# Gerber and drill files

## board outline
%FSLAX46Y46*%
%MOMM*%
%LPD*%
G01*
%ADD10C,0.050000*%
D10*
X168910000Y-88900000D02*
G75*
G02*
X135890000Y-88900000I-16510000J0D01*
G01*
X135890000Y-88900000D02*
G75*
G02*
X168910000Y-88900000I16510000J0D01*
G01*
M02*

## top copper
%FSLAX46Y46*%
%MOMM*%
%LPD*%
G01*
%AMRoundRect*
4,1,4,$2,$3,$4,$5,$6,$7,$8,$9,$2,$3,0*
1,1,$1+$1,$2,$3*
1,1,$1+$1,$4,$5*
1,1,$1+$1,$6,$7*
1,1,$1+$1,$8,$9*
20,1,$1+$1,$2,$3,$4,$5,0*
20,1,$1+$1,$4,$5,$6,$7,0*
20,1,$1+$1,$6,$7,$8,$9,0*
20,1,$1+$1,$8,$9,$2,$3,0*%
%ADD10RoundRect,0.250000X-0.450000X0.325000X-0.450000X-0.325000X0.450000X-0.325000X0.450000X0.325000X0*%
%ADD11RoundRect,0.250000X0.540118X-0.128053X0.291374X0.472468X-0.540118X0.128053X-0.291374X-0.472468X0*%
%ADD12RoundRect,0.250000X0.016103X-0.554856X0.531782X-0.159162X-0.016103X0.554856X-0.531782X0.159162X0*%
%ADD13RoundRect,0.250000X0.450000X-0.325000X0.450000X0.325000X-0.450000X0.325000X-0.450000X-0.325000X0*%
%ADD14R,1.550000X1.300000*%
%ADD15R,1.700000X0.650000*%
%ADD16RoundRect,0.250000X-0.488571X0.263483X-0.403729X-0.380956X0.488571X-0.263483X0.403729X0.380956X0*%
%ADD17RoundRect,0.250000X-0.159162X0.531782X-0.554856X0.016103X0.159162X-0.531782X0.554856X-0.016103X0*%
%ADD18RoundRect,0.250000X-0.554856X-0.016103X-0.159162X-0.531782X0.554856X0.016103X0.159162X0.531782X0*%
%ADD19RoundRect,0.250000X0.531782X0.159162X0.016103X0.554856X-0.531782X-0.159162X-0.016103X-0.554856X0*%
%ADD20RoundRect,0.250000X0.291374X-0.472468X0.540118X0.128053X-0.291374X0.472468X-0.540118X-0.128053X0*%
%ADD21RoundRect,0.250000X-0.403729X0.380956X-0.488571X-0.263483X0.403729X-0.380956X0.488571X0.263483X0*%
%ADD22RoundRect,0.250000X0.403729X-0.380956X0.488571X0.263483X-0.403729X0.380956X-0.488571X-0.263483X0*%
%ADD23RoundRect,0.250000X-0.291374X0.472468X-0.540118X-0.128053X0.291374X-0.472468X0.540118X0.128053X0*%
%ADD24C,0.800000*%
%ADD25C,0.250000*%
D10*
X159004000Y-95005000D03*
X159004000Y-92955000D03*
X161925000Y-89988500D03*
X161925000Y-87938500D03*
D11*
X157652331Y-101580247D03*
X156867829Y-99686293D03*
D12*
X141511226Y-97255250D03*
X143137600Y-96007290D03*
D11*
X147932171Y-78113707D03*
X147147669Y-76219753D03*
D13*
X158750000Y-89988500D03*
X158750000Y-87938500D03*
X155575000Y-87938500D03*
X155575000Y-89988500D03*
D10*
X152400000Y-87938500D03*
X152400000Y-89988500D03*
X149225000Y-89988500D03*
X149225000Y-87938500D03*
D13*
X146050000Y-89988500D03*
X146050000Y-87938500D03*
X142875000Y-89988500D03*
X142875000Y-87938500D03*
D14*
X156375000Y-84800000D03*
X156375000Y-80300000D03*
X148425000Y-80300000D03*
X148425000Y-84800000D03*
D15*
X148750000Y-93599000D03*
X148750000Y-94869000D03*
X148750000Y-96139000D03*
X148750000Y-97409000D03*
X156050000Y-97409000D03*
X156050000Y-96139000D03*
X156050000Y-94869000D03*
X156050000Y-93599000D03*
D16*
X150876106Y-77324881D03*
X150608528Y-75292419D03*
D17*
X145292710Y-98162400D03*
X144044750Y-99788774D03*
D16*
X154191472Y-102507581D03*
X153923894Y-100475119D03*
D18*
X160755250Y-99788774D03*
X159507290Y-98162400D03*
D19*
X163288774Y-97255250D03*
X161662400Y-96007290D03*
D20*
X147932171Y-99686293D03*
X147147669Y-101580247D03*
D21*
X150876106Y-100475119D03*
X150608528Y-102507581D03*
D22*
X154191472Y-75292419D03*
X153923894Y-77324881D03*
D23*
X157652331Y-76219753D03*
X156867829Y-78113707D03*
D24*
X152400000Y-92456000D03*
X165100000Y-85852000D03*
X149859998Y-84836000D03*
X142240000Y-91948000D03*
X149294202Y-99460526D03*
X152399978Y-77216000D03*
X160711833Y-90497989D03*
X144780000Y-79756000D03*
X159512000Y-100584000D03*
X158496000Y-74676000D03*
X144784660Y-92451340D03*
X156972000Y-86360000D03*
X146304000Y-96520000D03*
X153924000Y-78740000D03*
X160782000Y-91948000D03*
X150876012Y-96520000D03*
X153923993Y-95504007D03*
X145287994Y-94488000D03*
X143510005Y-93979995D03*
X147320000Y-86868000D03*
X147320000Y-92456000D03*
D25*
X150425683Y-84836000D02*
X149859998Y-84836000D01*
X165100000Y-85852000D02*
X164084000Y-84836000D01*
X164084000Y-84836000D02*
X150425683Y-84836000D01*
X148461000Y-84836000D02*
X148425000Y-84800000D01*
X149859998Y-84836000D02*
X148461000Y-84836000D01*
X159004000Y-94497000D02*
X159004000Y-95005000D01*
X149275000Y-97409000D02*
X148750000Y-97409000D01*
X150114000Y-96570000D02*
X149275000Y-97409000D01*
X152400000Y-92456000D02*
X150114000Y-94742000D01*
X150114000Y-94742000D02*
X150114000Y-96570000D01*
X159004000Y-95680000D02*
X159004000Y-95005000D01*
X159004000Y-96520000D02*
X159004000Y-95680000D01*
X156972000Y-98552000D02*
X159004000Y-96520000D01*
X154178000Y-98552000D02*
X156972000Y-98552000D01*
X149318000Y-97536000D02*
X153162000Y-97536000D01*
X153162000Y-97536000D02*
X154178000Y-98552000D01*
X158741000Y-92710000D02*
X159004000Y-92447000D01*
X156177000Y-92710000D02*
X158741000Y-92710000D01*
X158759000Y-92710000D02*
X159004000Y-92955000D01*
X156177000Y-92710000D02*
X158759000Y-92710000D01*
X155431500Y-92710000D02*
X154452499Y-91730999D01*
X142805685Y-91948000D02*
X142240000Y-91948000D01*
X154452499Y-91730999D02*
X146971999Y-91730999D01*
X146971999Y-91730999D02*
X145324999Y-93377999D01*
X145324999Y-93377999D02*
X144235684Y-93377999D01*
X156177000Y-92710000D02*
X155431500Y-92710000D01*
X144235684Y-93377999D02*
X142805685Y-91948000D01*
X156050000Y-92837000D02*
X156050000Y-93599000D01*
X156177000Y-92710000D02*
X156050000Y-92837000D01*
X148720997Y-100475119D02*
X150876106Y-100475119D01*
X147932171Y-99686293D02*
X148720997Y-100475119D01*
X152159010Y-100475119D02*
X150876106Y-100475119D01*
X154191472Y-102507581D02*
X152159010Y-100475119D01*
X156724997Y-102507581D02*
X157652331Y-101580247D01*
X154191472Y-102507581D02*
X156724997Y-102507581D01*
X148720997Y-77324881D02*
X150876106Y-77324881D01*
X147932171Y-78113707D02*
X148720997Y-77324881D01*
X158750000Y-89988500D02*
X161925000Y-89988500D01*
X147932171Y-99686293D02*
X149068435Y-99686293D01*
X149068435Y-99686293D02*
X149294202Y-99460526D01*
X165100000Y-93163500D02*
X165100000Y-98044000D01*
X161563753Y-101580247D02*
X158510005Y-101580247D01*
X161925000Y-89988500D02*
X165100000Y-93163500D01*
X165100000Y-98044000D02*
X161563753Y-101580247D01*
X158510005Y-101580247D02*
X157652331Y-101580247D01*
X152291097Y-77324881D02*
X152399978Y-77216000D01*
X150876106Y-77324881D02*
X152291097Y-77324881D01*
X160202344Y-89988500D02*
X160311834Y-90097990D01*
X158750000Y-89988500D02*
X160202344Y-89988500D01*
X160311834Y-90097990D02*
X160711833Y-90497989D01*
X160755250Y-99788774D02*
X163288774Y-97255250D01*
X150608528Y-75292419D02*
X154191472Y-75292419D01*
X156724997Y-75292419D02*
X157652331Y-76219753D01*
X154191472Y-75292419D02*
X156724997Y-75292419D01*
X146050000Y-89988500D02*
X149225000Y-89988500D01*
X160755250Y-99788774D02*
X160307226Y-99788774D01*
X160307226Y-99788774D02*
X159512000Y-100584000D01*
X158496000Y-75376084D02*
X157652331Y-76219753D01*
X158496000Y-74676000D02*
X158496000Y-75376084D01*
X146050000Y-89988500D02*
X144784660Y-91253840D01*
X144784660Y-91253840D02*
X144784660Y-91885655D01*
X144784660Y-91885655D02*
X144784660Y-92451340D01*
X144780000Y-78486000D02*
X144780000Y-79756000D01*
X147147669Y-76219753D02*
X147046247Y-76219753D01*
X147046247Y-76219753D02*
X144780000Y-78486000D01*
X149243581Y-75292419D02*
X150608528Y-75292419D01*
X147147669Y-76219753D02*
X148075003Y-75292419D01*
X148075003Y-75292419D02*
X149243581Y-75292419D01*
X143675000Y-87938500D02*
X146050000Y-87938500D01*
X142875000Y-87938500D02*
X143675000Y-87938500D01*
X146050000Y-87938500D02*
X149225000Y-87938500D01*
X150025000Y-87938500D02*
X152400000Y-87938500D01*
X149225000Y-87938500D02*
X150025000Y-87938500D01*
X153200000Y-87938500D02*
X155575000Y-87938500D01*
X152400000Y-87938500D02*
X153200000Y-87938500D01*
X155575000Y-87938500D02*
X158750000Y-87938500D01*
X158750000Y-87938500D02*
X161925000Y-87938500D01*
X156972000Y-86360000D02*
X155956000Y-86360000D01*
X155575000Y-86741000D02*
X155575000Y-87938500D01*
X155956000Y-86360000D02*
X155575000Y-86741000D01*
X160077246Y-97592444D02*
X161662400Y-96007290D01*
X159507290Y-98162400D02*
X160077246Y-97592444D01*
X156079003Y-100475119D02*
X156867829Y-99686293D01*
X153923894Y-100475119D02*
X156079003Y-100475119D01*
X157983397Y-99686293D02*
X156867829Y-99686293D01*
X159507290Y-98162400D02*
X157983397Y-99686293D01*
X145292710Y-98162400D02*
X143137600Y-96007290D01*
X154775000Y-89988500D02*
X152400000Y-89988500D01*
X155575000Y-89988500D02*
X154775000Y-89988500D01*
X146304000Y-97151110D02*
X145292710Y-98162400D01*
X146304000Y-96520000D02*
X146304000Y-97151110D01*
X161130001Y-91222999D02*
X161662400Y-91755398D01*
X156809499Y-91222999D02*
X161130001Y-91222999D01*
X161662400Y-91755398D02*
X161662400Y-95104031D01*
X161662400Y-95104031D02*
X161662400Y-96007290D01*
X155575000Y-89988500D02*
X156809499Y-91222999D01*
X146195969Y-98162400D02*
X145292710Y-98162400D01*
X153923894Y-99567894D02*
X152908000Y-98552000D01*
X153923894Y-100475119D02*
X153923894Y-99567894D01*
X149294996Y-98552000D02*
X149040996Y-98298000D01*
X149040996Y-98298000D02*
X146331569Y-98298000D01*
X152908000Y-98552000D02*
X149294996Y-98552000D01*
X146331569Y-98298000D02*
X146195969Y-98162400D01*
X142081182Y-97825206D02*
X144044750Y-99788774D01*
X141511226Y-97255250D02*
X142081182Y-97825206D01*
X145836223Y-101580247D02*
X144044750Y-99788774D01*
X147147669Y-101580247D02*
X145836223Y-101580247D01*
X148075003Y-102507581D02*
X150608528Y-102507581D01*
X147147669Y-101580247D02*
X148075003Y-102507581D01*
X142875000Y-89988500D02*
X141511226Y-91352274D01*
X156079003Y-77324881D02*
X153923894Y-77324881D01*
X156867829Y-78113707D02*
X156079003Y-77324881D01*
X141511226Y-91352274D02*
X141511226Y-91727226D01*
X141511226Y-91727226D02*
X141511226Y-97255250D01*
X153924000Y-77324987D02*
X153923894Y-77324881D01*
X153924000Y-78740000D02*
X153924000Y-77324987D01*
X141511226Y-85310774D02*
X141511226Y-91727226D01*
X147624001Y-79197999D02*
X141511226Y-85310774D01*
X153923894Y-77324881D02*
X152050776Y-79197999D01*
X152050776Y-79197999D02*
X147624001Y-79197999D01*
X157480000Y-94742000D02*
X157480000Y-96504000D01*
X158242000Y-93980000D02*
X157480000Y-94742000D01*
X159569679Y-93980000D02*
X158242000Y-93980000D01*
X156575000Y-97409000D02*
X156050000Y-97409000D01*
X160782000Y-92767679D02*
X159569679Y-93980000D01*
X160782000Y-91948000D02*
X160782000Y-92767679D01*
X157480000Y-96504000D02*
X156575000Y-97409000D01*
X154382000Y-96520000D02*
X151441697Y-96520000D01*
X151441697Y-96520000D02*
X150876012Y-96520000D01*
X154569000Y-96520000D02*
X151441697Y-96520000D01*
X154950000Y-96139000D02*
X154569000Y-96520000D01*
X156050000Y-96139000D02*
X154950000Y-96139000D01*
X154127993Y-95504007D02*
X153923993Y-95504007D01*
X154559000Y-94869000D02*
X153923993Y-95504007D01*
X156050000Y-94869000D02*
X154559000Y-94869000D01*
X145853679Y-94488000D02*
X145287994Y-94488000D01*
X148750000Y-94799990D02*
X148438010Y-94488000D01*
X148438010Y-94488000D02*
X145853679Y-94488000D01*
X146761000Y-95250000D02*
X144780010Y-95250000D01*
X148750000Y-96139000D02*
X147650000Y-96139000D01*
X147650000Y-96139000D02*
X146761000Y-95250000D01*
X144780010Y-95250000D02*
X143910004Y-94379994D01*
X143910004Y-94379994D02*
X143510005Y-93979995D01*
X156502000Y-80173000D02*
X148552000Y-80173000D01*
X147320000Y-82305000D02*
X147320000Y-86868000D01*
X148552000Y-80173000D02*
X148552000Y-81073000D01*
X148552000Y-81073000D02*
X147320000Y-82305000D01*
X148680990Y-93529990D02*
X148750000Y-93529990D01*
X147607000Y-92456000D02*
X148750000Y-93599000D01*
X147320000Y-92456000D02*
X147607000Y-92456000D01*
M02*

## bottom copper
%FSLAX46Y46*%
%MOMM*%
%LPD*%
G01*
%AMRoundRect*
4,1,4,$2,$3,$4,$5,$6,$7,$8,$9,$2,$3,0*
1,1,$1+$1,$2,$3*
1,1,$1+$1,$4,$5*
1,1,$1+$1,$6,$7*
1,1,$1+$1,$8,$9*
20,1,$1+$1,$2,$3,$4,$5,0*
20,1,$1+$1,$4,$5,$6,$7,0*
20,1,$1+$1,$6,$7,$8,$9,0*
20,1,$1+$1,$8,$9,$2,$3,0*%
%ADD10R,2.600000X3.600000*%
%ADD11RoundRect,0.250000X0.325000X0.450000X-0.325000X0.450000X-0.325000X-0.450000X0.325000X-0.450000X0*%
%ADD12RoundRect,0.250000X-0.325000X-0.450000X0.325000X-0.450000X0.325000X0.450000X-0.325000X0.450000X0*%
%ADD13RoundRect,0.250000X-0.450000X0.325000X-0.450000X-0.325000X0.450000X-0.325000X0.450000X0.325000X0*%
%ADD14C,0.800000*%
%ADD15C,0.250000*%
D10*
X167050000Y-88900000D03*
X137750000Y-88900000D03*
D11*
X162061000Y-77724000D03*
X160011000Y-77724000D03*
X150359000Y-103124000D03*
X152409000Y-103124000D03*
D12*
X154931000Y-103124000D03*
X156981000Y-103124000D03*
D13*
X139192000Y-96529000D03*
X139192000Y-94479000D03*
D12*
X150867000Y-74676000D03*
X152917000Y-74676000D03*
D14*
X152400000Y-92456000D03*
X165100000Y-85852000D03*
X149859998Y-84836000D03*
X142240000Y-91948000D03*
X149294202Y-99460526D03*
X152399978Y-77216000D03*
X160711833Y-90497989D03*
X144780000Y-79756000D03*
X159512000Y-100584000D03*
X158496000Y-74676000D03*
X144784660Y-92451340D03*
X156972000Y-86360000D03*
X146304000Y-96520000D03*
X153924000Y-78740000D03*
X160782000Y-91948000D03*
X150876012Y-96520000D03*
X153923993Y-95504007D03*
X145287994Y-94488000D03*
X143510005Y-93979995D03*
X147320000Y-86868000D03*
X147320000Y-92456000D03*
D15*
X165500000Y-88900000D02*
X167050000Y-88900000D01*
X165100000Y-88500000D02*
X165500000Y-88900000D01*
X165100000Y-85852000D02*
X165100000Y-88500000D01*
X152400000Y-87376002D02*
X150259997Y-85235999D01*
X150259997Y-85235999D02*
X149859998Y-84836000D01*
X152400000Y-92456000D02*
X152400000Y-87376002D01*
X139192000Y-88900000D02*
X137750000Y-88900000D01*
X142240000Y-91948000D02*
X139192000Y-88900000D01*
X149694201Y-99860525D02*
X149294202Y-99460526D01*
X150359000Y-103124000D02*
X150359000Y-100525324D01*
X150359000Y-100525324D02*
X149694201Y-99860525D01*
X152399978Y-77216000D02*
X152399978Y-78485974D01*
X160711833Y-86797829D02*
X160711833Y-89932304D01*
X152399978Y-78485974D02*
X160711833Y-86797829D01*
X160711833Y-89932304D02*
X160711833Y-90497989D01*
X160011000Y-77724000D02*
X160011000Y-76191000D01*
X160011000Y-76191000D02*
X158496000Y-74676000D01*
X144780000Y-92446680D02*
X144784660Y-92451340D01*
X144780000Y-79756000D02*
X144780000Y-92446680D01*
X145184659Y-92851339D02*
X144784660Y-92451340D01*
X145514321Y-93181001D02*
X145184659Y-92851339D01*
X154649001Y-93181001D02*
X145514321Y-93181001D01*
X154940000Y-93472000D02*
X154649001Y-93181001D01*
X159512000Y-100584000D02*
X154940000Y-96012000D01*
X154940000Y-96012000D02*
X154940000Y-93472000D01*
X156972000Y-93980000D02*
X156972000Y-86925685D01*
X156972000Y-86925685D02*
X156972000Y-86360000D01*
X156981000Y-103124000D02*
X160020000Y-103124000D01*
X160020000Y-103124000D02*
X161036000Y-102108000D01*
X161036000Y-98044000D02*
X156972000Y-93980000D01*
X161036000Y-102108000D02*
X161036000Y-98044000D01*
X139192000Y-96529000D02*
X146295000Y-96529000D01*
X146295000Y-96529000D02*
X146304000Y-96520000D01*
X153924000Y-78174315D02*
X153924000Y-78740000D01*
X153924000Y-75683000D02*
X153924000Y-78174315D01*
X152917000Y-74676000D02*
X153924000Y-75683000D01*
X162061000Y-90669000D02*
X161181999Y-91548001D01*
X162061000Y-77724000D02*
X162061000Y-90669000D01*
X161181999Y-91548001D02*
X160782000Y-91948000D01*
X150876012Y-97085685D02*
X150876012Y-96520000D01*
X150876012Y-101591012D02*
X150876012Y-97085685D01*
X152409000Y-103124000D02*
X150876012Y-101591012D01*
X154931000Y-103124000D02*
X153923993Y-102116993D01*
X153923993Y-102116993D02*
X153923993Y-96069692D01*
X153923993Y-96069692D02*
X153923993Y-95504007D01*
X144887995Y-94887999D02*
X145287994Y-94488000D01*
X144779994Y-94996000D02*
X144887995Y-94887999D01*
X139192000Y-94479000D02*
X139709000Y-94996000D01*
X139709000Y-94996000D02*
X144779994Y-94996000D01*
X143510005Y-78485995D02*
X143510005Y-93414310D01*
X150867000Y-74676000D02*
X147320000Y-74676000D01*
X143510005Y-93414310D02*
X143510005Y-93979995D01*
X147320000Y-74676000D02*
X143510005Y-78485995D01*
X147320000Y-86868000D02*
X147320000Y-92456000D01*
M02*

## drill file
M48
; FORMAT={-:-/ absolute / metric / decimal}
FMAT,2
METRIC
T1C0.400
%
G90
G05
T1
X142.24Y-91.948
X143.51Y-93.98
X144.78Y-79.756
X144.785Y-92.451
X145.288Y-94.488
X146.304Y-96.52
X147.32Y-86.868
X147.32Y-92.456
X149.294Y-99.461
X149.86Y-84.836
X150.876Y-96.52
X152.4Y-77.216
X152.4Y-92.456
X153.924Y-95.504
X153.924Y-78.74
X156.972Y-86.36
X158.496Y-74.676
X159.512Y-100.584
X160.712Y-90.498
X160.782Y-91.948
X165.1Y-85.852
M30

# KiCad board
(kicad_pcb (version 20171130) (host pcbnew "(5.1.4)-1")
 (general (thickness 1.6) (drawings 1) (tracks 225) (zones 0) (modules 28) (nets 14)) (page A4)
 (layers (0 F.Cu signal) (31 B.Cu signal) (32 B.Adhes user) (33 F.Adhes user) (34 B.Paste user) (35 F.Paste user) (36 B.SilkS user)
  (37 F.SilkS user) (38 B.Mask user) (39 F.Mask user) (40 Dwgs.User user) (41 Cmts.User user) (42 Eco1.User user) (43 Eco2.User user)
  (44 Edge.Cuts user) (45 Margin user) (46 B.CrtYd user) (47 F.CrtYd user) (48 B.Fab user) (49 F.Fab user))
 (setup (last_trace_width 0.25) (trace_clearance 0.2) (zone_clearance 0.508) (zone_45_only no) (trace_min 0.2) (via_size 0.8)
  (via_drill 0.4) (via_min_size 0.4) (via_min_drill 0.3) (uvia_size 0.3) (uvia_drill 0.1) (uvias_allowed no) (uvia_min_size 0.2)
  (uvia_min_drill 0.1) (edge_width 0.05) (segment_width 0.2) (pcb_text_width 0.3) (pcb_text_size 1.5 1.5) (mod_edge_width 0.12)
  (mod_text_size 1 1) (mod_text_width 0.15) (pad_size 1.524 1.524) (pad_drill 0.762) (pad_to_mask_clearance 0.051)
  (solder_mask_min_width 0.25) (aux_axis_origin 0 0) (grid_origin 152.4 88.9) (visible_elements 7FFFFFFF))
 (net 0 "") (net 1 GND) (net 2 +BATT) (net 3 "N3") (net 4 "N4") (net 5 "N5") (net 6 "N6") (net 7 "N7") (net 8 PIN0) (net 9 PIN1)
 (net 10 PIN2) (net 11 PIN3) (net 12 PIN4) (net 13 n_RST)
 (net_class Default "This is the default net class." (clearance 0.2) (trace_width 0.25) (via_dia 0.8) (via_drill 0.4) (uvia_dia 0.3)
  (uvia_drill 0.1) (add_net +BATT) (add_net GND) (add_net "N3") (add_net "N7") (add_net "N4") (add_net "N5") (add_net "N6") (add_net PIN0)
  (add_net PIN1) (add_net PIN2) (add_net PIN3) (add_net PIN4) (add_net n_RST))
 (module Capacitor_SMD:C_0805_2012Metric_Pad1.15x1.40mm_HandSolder (layer F.Cu) (at 159.004 93.98 270)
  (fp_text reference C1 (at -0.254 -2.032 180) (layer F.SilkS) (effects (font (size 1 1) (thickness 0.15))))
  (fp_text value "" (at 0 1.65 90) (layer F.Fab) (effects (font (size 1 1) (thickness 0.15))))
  (pad 2 smd roundrect (at 1.025 0 270) (size 1.15 1.4) (layers F.Cu F.Paste F.Mask) (roundrect_rratio 0.217391) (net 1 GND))
  (pad 1 smd roundrect (at -1.025 0 270) (size 1.15 1.4) (layers F.Cu F.Paste F.Mask) (roundrect_rratio 0.217391) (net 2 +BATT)))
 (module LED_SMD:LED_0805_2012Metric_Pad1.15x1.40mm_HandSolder (layer F.Cu) (at 161.925 88.9635 270)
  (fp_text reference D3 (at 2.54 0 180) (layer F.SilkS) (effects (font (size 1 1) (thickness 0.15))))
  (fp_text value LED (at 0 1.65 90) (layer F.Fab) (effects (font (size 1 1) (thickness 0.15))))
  (pad 2 smd roundrect (at 1.025 0 270) (size 1.15 1.4) (layers F.Cu F.Paste F.Mask) (roundrect_rratio 0.217391) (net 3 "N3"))
  (pad 1 smd roundrect (at -1.025 0 270) (size 1.15 1.4) (layers F.Cu F.Paste F.Mask) (roundrect_rratio 0.217391) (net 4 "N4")))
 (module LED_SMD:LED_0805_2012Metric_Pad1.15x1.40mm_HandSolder (layer F.Cu) (at 157.26008 100.63327 112.5)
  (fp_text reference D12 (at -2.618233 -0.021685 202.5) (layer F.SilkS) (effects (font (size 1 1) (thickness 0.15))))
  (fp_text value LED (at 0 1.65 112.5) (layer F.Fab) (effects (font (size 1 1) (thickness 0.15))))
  (pad 1 smd roundrect (at -1.025 0 112.5) (size 1.15 1.4) (layers F.Cu F.Paste F.Mask) (roundrect_rratio 0.217391) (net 3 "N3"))
  (pad 2 smd roundrect (at 1.025 0 112.5) (size 1.15 1.4) (layers F.Cu F.Paste F.Mask) (roundrect_rratio 0.217391) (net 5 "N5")))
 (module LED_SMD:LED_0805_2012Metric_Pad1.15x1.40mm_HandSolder (layer F.Cu) (at 142.324413 96.63127 37.5)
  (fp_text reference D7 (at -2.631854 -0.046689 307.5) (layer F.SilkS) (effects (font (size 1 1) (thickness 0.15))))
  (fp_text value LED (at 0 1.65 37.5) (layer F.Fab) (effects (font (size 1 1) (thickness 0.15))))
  (pad 1 smd roundrect (at -1.025 0 37.5) (size 1.15 1.4) (layers F.Cu F.Paste F.Mask) (roundrect_rratio 0.217391) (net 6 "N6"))
  (pad 2 smd roundrect (at 1.025 0 37.5) (size 1.15 1.4) (layers F.Cu F.Paste F.Mask) (roundrect_rratio 0.217391) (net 5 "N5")))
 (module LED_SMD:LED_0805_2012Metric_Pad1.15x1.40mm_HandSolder (layer F.Cu) (at 147.53992 77.16673 112.5)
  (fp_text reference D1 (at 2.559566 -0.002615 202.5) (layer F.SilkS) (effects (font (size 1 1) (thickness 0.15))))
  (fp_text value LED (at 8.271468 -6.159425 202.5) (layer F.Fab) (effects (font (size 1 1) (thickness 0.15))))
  (pad 1 smd roundrect (at -1.025 0 112.5) (size 1.15 1.4) (layers F.Cu F.Paste F.Mask) (roundrect_rratio 0.217391) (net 3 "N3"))
  (pad 2 smd roundrect (at 1.025 0 112.5) (size 1.15 1.4) (layers F.Cu F.Paste F.Mask) (roundrect_rratio 0.217391) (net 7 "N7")))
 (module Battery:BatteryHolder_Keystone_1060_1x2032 (layer B.Cu) (at 152.4 88.9)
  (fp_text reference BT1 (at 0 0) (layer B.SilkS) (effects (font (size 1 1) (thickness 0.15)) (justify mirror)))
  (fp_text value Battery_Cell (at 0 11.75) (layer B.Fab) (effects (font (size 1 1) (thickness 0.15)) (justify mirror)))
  (pad 2 smd rect (at 14.65 0 180) (size 2.6 3.6) (layers B.Cu B.Paste B.Mask) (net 1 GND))
  (pad 1 smd rect (at -14.65 0 180) (size 2.6 3.6) (layers B.Cu B.Paste B.Mask) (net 2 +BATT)))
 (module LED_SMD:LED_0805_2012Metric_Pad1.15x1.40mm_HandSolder (layer F.Cu) (at 158.75 88.9635 90)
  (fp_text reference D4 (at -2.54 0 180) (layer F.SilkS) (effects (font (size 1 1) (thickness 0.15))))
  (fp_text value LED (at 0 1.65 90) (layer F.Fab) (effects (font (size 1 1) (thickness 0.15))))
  (pad 1 smd roundrect (at -1.025 0 90) (size 1.15 1.4) (layers F.Cu F.Paste F.Mask) (roundrect_rratio 0.217391) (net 3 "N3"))
  (pad 2 smd roundrect (at 1.025 0 90) (size 1.15 1.4) (layers F.Cu F.Paste F.Mask) (roundrect_rratio 0.217391) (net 4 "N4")))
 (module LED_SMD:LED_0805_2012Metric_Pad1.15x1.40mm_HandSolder (layer F.Cu) (at 155.575 88.9635 90)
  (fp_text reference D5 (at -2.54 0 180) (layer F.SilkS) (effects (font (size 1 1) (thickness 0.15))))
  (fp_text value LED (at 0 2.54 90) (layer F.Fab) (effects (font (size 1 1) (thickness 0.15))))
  (pad 2 smd roundrect (at 1.025 0 90) (size 1.15 1.4) (layers F.Cu F.Paste F.Mask) (roundrect_rratio 0.217391) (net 4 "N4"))
  (pad 1 smd roundrect (at -1.025 0 90) (size 1.15 1.4) (layers F.Cu F.Paste F.Mask) (roundrect_rratio 0.217391) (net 5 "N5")))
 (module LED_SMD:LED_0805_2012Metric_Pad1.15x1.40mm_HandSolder (layer F.Cu) (at 152.4 88.9635 270)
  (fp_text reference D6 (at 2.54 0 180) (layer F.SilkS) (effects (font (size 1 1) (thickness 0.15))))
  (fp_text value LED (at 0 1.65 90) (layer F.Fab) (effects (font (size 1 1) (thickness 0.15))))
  (pad 1 smd roundrect (at -1.025 0 270) (size 1.15 1.4) (layers F.Cu F.Paste F.Mask) (roundrect_rratio 0.217391) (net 4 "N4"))
  (pad 2 smd roundrect (at 1.025 0 270) (size 1.15 1.4) (layers F.Cu F.Paste F.Mask) (roundrect_rratio 0.217391) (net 5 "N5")))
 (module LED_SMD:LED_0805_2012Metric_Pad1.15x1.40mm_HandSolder (layer F.Cu) (at 149.225 88.9635 270)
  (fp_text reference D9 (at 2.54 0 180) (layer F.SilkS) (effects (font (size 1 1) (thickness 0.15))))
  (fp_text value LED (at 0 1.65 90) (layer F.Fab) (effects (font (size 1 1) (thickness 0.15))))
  (pad 2 smd roundrect (at 1.025 0 270) (size 1.15 1.4) (layers F.Cu F.Paste F.Mask) (roundrect_rratio 0.217391) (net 7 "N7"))
  (pad 1 smd roundrect (at -1.025 0 270) (size 1.15 1.4) (layers F.Cu F.Paste F.Mask) (roundrect_rratio 0.217391) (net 4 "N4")))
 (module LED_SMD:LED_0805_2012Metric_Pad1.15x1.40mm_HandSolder (layer F.Cu) (at 146.05 88.9635 90)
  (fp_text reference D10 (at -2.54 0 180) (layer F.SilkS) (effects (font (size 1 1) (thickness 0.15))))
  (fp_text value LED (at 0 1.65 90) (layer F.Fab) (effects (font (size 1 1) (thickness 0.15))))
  (pad 1 smd roundrect (at -1.025 0 90) (size 1.15 1.4) (layers F.Cu F.Paste F.Mask) (roundrect_rratio 0.217391) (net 7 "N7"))
  (pad 2 smd roundrect (at 1.025 0 90) (size 1.15 1.4) (layers F.Cu F.Paste F.Mask) (roundrect_rratio 0.217391) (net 4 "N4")))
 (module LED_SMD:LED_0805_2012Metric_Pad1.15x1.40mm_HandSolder (layer F.Cu) (at 142.875 88.9635 90)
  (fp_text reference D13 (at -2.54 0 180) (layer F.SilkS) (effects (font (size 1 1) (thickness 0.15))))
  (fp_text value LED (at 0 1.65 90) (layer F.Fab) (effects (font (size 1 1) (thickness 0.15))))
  (pad 1 smd roundrect (at -1.025 0 90) (size 1.15 1.4) (layers F.Cu F.Paste F.Mask) (roundrect_rratio 0.217391) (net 6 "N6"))
  (pad 2 smd roundrect (at 1.025 0 90) (size 1.15 1.4) (layers F.Cu F.Paste F.Mask) (roundrect_rratio 0.217391) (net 4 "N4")))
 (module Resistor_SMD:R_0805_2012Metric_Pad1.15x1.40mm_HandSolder (layer B.Cu) (at 161.036 77.724 180)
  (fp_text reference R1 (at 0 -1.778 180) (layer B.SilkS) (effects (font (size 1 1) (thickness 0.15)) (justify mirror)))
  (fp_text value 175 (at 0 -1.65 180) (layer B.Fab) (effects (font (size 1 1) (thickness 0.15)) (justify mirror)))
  (pad 1 smd roundrect (at -1.025 0 180) (size 1.15 1.4) (layers B.Cu B.Paste B.Mask) (roundrect_rratio 0.217391) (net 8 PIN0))
  (pad 2 smd roundrect (at 1.025 0 180) (size 1.15 1.4) (layers B.Cu B.Paste B.Mask) (roundrect_rratio 0.217391) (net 7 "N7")))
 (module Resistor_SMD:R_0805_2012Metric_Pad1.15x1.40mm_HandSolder (layer B.Cu) (at 151.384 103.124 180)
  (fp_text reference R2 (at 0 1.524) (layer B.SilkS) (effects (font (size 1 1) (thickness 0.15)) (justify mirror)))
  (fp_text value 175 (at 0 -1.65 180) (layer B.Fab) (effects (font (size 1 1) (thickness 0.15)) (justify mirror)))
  (pad 2 smd roundrect (at 1.025 0 180) (size 1.15 1.4) (layers B.Cu B.Paste B.Mask) (roundrect_rratio 0.217391) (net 3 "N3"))
  (pad 1 smd roundrect (at -1.025 0 180) (size 1.15 1.4) (layers B.Cu B.Paste B.Mask) (roundrect_rratio 0.217391) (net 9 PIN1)))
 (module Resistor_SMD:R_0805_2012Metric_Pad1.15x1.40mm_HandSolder (layer B.Cu) (at 155.956 103.124)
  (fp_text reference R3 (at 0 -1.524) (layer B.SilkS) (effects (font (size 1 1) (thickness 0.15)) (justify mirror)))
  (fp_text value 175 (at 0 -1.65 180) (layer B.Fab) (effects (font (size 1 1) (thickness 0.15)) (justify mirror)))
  (pad 1 smd roundrect (at -1.025 0) (size 1.15 1.4) (layers B.Cu B.Paste B.Mask) (roundrect_rratio 0.217391) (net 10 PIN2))
  (pad 2 smd roundrect (at 1.025 0) (size 1.15 1.4) (layers B.Cu B.Paste B.Mask) (roundrect_rratio 0.217391) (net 4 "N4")))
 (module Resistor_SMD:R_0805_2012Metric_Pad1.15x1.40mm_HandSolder (layer B.Cu) (at 139.192 95.504 270)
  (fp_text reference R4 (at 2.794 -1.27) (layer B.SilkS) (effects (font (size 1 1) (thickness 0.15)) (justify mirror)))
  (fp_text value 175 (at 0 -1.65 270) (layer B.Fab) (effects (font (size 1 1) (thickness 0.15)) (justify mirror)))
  (pad 2 smd roundrect (at 1.025 0 270) (size 1.15 1.4) (layers B.Cu B.Paste B.Mask) (roundrect_rratio 0.217391) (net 5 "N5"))
  (pad 1 smd roundrect (at -1.025 0 270) (size 1.15 1.4) (layers B.Cu B.Paste B.Mask) (roundrect_rratio 0.217391) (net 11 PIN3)))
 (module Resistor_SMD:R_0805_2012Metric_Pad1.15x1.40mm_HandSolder (layer B.Cu) (at 151.892 74.676)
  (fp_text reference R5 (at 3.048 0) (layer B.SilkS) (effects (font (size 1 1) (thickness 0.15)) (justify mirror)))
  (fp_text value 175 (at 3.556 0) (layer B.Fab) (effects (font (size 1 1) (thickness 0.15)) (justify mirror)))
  (pad 1 smd roundrect (at -1.025 0) (size 1.15 1.4) (layers B.Cu B.Paste B.Mask) (roundrect_rratio 0.217391) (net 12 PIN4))
  (pad 2 smd roundrect (at 1.025 0) (size 1.15 1.4) (layers B.Cu B.Paste B.Mask) (roundrect_rratio 0.217391) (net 6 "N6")))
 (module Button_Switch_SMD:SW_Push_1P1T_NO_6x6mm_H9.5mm (layer F.Cu) (at 152.4 82.55)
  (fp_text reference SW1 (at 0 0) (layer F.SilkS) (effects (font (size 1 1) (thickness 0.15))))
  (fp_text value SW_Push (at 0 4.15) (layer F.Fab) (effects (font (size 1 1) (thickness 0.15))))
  (pad 2 smd rect (at 3.975 2.25) (size 1.55 1.3) (layers F.Cu F.Paste F.Mask) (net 1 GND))
  (pad 1 smd rect (at 3.975 -2.25) (size 1.55 1.3) (layers F.Cu F.Paste F.Mask) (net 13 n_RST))
  (pad 1 smd rect (at -3.975 -2.25) (size 1.55 1.3) (layers F.Cu F.Paste F.Mask) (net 13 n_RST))
  (pad 2 smd rect (at -3.975 2.25) (size 1.55 1.3) (layers F.Cu F.Paste F.Mask) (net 1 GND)))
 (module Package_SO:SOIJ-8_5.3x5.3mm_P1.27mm (layer F.Cu) (at 152.4 95.504)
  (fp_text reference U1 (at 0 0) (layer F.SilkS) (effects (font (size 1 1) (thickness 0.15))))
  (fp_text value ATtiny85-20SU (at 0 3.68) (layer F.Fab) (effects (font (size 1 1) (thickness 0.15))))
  (pad 1 smd rect (at -3.65 -1.905) (size 1.7 0.65) (layers F.Cu F.Paste F.Mask) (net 13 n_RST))
  (pad 2 smd rect (at -3.65 -0.635) (size 1.7 0.65) (layers F.Cu F.Paste F.Mask) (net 11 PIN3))
  (pad 3 smd rect (at -3.65 0.635) (size 1.7 0.65) (layers F.Cu F.Paste F.Mask) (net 12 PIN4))
  (pad 4 smd rect (at -3.65 1.905) (size 1.7 0.65) (layers F.Cu F.Paste F.Mask) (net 1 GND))
  (pad 5 smd rect (at 3.65 1.905) (size 1.7 0.65) (layers F.Cu F.Paste F.Mask) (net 8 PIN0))
  (pad 6 smd rect (at 3.65 0.635) (size 1.7 0.65) (layers F.Cu F.Paste F.Mask) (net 9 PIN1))
  (pad 7 smd rect (at 3.65 -0.635) (size 1.7 0.65) (layers F.Cu F.Paste F.Mask) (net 10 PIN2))
  (pad 8 smd rect (at 3.65 -1.905) (size 1.7 0.65) (layers F.Cu F.Paste F.Mask) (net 2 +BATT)))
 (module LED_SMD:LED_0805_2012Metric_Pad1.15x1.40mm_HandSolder (layer F.Cu) (at 150.742317 76.30865 277.5)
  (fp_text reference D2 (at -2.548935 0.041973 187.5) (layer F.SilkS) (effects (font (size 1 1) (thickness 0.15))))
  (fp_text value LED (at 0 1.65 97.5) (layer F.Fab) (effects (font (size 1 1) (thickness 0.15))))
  (pad 2 smd roundrect (at 1.025 0 277.5) (size 1.15 1.4) (layers F.Cu F.Paste F.Mask) (roundrect_rratio 0.217391) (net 3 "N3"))
  (pad 1 smd roundrect (at -1.025 0 277.5) (size 1.15 1.4) (layers F.Cu F.Paste F.Mask) (roundrect_rratio 0.217391) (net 7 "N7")))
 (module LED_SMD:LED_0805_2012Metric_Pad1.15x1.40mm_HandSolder (layer F.Cu) (at 144.66873 98.975587 232.5)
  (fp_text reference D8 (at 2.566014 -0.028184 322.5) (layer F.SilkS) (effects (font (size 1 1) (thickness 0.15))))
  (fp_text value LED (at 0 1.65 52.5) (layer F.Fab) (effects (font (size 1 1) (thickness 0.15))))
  (pad 1 smd roundrect (at -1.025 0 232.5) (size 1.15 1.4) (layers F.Cu F.Paste F.Mask) (roundrect_rratio 0.217391) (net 5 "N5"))
  (pad 2 smd roundrect (at 1.025 0 232.5) (size 1.15 1.4) (layers F.Cu F.Paste F.Mask) (roundrect_rratio 0.217391) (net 6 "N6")))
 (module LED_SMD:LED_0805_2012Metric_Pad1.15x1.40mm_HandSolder (layer F.Cu) (at 154.057683 101.49135 277.5)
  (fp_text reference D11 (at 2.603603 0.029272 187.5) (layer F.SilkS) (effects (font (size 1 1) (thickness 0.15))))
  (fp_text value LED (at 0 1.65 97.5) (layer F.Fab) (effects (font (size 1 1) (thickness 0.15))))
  (pad 2 smd roundrect (at 1.025 0 277.5) (size 1.15 1.4) (layers F.Cu F.Paste F.Mask) (roundrect_rratio 0.217391) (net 3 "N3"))
  (pad 1 smd roundrect (at -1.025 0 277.5) (size 1.15 1.4) (layers F.Cu F.Paste F.Mask) (roundrect_rratio 0.217391) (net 5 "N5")))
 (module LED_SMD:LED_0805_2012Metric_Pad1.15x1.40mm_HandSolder (layer F.Cu) (at 160.13127 98.975587 307.5)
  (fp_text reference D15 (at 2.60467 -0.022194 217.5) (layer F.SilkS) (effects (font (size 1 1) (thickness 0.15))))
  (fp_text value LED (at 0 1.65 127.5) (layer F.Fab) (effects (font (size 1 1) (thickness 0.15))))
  (pad 2 smd roundrect (at 1.025 0 307.5) (size 1.15 1.4) (layers F.Cu F.Paste F.Mask) (roundrect_rratio 0.217391) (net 7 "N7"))
  (pad 1 smd roundrect (at -1.025 0 307.5) (size 1.15 1.4) (layers F.Cu F.Paste F.Mask) (roundrect_rratio 0.217391) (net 5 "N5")))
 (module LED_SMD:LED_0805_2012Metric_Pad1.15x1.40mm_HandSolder (layer F.Cu) (at 162.475587 96.63127 142.5)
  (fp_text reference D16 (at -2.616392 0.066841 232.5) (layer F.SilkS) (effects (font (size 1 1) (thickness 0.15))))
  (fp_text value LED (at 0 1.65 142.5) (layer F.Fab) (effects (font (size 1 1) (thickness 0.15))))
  (pad 1 smd roundrect (at -1.025 0 142.5) (size 1.15 1.4) (layers F.Cu F.Paste F.Mask) (roundrect_rratio 0.217391) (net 7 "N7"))
  (pad 2 smd roundrect (at 1.025 0 142.5) (size 1.15 1.4) (layers F.Cu F.Paste F.Mask) (roundrect_rratio 0.217391) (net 5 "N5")))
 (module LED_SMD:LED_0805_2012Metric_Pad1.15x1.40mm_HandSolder (layer F.Cu) (at 147.53992 100.63327 67.5)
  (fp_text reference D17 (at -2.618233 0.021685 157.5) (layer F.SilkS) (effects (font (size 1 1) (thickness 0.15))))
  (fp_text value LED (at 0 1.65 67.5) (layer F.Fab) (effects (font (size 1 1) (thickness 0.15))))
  (pad 2 smd roundrect (at 1.025 0 67.5) (size 1.15 1.4) (layers F.Cu F.Paste F.Mask) (roundrect_rratio 0.217391) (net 3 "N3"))
  (pad 1 smd roundrect (at -1.025 0 67.5) (size 1.15 1.4) (layers F.Cu F.Paste F.Mask) (roundrect_rratio 0.217391) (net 6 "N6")))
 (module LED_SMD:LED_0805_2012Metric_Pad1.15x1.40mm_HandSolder (layer F.Cu) (at 150.742317 101.49135 262.5)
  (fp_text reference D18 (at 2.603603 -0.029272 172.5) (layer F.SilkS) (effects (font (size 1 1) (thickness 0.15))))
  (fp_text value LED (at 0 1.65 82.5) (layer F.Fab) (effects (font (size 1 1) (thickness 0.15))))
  (pad 1 smd roundrect (at -1.025 0 262.5) (size 1.15 1.4) (layers F.Cu F.Paste F.Mask) (roundrect_rratio 0.217391) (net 3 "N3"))
  (pad 2 smd roundrect (at 1.025 0 262.5) (size 1.15 1.4) (layers F.Cu F.Paste F.Mask) (roundrect_rratio 0.217391) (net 6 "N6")))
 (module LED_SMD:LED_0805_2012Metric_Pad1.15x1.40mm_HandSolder (layer F.Cu) (at 154.057683 76.30865 82.5)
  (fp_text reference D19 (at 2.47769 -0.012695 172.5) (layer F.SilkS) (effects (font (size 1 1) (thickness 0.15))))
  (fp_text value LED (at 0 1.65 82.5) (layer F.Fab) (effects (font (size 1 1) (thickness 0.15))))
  (pad 2 smd roundrect (at 1.025 0 82.5) (size 1.15 1.4) (layers F.Cu F.Paste F.Mask) (roundrect_rratio 0.217391) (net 7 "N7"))
  (pad 1 smd roundrect (at -1.025 0 82.5) (size 1.15 1.4) (layers F.Cu F.Paste F.Mask) (roundrect_rratio 0.217391) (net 6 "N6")))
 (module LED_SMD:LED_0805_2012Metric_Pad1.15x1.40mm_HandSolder (layer F.Cu) (at 157.26008 77.16673 247.5)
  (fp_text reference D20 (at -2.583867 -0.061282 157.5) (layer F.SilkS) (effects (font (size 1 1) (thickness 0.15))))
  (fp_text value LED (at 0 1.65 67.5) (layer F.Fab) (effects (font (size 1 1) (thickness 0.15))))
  (pad 1 smd roundrect (at -1.025 0 247.5) (size 1.15 1.4) (layers F.Cu F.Paste F.Mask) (roundrect_rratio 0.217391) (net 7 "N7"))
  (pad 2 smd roundrect (at 1.025 0 247.5) (size 1.15 1.4) (layers F.Cu F.Paste F.Mask) (roundrect_rratio 0.217391) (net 6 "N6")))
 (gr_circle (center 152.4 88.9) (end 168.91 88.9) (layer Edge.Cuts) (width 0.05))
 (via (at 152.4 92.456) (size 0.8) (drill 0.4) (layers F.Cu B.Cu) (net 1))
 (via (at 165.1 85.852) (size 0.8) (drill 0.4) (layers F.Cu B.Cu) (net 1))
 (segment (start 165.5 88.9) (end 167.05 88.9) (width 0.25) (layer B.Cu) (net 1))
 (segment (start 165.1 88.5) (end 165.5 88.9) (width 0.25) (layer B.Cu) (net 1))
 (segment (start 165.1 85.852) (end 165.1 88.5) (width 0.25) (layer B.Cu) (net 1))
 (via (at 149.859998 84.836) (size 0.8) (drill 0.4) (layers F.Cu B.Cu) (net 1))
 (segment (start 152.4 87.376002) (end 150.259997 85.235999) (width 0.25) (layer B.Cu) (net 1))
 (segment (start 150.259997 85.235999) (end 149.859998 84.836) (width 0.25) (layer B.Cu) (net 1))
 (segment (start 152.4 92.456) (end 152.4 87.376002) (width 0.25) (layer B.Cu) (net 1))
 (segment (start 150.425683 84.836) (end 149.859998 84.836) (width 0.25) (layer F.Cu) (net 1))
 (segment (start 165.1 85.852) (end 164.084 84.836) (width 0.25) (layer F.Cu) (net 1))
 (segment (start 164.084 84.836) (end 150.425683 84.836) (width 0.25) (layer F.Cu) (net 1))
 (segment (start 148.461 84.836) (end 148.425 84.8) (width 0.25) (layer F.Cu) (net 1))
 (segment (start 149.859998 84.836) (end 148.461 84.836) (width 0.25) (layer F.Cu) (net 1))
 (segment (start 159.004 94.497) (end 159.004 95.005) (width 0.25) (layer F.Cu) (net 1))
 (segment (start 149.275 97.409) (end 148.75 97.409) (width 0.25) (layer F.Cu) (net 1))
 (segment (start 150.114 96.57) (end 149.275 97.409) (width 0.25) (layer F.Cu) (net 1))
 (segment (start 152.4 92.456) (end 150.114 94.742) (width 0.25) (layer F.Cu) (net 1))
 (segment (start 150.114 94.742) (end 150.114 96.57) (width 0.25) (layer F.Cu) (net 1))
 (segment (start 159.004 95.68) (end 159.004 95.005) (width 0.25) (layer F.Cu) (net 1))
 (segment (start 159.004 96.52) (end 159.004 95.68) (width 0.25) (layer F.Cu) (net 1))
 (segment (start 156.972 98.552) (end 159.004 96.52) (width 0.25) (layer F.Cu) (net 1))
 (segment (start 154.178 98.552) (end 156.972 98.552) (width 0.25) (layer F.Cu) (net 1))
 (segment (start 149.318 97.536) (end 153.162 97.536) (width 0.25) (layer F.Cu) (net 1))
 (segment (start 153.162 97.536) (end 154.178 98.552) (width 0.25) (layer F.Cu) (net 1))
 (via (at 142.24 91.948) (size 0.8) (drill 0.4) (layers F.Cu B.Cu) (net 2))
 (segment (start 139.192 88.9) (end 137.75 88.9) (width 0.25) (layer B.Cu) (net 2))
 (segment (start 142.24 91.948) (end 139.192 88.9) (width 0.25) (layer B.Cu) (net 2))
 (segment (start 158.741 92.71) (end 159.004 92.447) (width 0.25) (layer F.Cu) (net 2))
 (segment (start 156.177 92.71) (end 158.741 92.71) (width 0.25) (layer F.Cu) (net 2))
 (segment (start 158.759 92.71) (end 159.004 92.955) (width 0.25) (layer F.Cu) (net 2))
 (segment (start 156.177 92.71) (end 158.759 92.71) (width 0.25) (layer F.Cu) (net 2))
 (segment (start 155.4315 92.71) (end 154.452499 91.730999) (width 0.25) (layer F.Cu) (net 2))
 (segment (start 142.805685 91.948) (end 142.24 91.948) (width 0.25) (layer F.Cu) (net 2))
 (segment (start 154.452499 91.730999) (end 146.971999 91.730999) (width 0.25) (layer F.Cu) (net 2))
 (segment (start 146.971999 91.730999) (end 145.324999 93.377999) (width 0.25) (layer F.Cu) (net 2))
 (segment (start 145.324999 93.377999) (end 144.235684 93.377999) (width 0.25) (layer F.Cu) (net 2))
 (segment (start 156.177 92.71) (end 155.4315 92.71) (width 0.25) (layer F.Cu) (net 2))
 (segment (start 144.235684 93.377999) (end 142.805685 91.948) (width 0.25) (layer F.Cu) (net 2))
 (segment (start 156.05 92.837) (end 156.05 93.599) (width 0.25) (layer F.Cu) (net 2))
 (segment (start 156.177 92.71) (end 156.05 92.837) (width 0.25) (layer F.Cu) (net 2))
 (segment (start 148.720997 100.475119) (end 150.876106 100.475119) (width 0.25) (layer F.Cu) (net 3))
 (segment (start 147.932171 99.686293) (end 148.720997 100.475119) (width 0.25) (layer F.Cu) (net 3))
 (segment (start 152.15901 100.475119) (end 150.876106 100.475119) (width 0.25) (layer F.Cu) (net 3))
 (segment (start 154.191472 102.507581) (end 152.15901 100.475119) (width 0.25) (layer F.Cu) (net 3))
 (segment (start 156.724997 102.507581) (end 157.652331 101.580247) (width 0.25) (layer F.Cu) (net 3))
 (segment (start 154.191472 102.507581) (end 156.724997 102.507581) (width 0.25) (layer F.Cu) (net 3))
 (segment (start 148.720997 77.324881) (end 150.876106 77.324881) (width 0.25) (layer F.Cu) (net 3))
 (segment (start 147.932171 78.113707) (end 148.720997 77.324881) (width 0.25) (layer F.Cu) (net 3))
 (segment (start 158.75 89.9885) (end 161.925 89.9885) (width 0.25) (layer F.Cu) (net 3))
 (segment (start 149.694201 99.860525) (end 149.294202 99.460526) (width 0.25) (layer B.Cu) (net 3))
 (segment (start 150.359 103.124) (end 150.359 100.525324) (width 0.25) (layer B.Cu) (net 3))
 (segment (start 150.359 100.525324) (end 149.694201 99.860525) (width 0.25) (layer B.Cu) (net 3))
 (via (at 149.294202 99.460526) (size 0.8) (drill 0.4) (layers F.Cu B.Cu) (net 3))
 (segment (start 147.932171 99.686293) (end 149.068435 99.686293) (width 0.25) (layer F.Cu) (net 3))
 (segment (start 149.068435 99.686293) (end 149.294202 99.460526) (width 0.25) (layer F.Cu) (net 3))
 (segment (start 165.1 93.1635) (end 165.1 98.044) (width 0.25) (layer F.Cu) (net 3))
 (segment (start 161.563753 101.580247) (end 158.510005 101.580247) (width 0.25) (layer F.Cu) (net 3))
 (segment (start 161.925 89.9885) (end 165.1 93.1635) (width 0.25) (layer F.Cu) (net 3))
 (segment (start 165.1 98.044) (end 161.563753 101.580247) (width 0.25) (layer F.Cu) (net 3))
 (segment (start 158.510005 101.580247) (end 157.652331 101.580247) (width 0.25) (layer F.Cu) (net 3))
 (via (at 152.399978 77.216) (size 0.8) (drill 0.4) (layers F.Cu B.Cu) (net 3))
 (segment (start 152.291097 77.324881) (end 152.399978 77.216) (width 0.25) (layer F.Cu) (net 3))
 (segment (start 150.876106 77.324881) (end 152.291097 77.324881) (width 0.25) (layer F.Cu) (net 3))
 (segment (start 152.399978 77.216) (end 152.399978 78.485974) (width 0.25) (layer B.Cu) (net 3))
 (segment (start 160.711833 86.797829) (end 160.711833 89.932304) (width 0.25) (layer B.Cu) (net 3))
 (via (at 160.711833 90.497989) (size 0.8) (drill 0.4) (layers F.Cu B.Cu) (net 3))
 (segment (start 160.202344 89.9885) (end 160.311834 90.09799) (width 0.25) (layer F.Cu) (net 3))
 (segment (start 152.399978 78.485974) (end 160.711833 86.797829) (width 0.25) (layer B.Cu) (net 3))
 (segment (start 158.75 89.9885) (end 160.202344 89.9885) (width 0.25) (layer F.Cu) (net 3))
 (segment (start 160.311834 90.09799) (end 160.711833 90.497989) (width 0.25) (layer F.Cu) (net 3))
 (segment (start 160.711833 89.932304) (end 160.711833 90.497989) (width 0.25) (layer B.Cu) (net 3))
 (segment (start 160.75525 99.788774) (end 163.288774 97.25525) (width 0.25) (layer F.Cu) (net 7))
 (segment (start 150.608528 75.292419) (end 154.191472 75.292419) (width 0.25) (layer F.Cu) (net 7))
 (segment (start 156.724997 75.292419) (end 157.652331 76.219753) (width 0.25) (layer F.Cu) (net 7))
 (segment (start 154.191472 75.292419) (end 156.724997 75.292419) (width 0.25) (layer F.Cu) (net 7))
 (segment (start 146.05 89.9885) (end 149.225 89.9885) (width 0.25) (layer F.Cu) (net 7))
 (via (at 144.78 79.756) (size 0.8) (drill 0.4) (layers F.Cu B.Cu) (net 7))
 (via (at 159.512 100.584) (size 0.8) (drill 0.4) (layers F.Cu B.Cu) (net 7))
 (segment (start 160.75525 99.788774) (end 160.307226 99.788774) (width 0.25) (layer F.Cu) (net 7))
 (segment (start 160.307226 99.788774) (end 159.512 100.584) (width 0.25) (layer F.Cu) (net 7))
 (via (at 158.496 74.676) (size 0.8) (drill 0.4) (layers F.Cu B.Cu) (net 7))
 (segment (start 160.011 77.724) (end 160.011 76.191) (width 0.25) (layer B.Cu) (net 7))
 (segment (start 160.011 76.191) (end 158.496 74.676) (width 0.25) (layer B.Cu) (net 7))
 (segment (start 158.496 75.376084) (end 157.652331 76.219753) (width 0.25) (layer F.Cu) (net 7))
 (segment (start 158.496 74.676) (end 158.496 75.376084) (width 0.25) (layer F.Cu) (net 7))
 (segment (start 146.05 89.9885) (end 144.78466 91.25384) (width 0.25) (layer F.Cu) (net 7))
 (segment (start 144.78466 91.25384) (end 144.78466 91.885655) (width 0.25) (layer F.Cu) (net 7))
 (via (at 144.78466 92.45134) (size 0.8) (drill 0.4) (layers F.Cu B.Cu) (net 7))
 (segment (start 144.78 92.44668) (end 144.78466 92.45134) (width 0.25) (layer B.Cu) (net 7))
 (segment (start 144.78 79.756) (end 144.78 92.44668) (width 0.25) (layer B.Cu) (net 7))
 (segment (start 144.78466 91.885655) (end 144.78466 92.45134) (width 0.25) (layer F.Cu) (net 7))
 (segment (start 145.184659 92.851339) (end 144.78466 92.45134) (width 0.25) (layer B.Cu) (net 7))
 (segment (start 145.514321 93.181001) (end 145.184659 92.851339) (width 0.25) (layer B.Cu) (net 7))
 (segment (start 154.649001 93.181001) (end 145.514321 93.181001) (width 0.25) (layer B.Cu) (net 7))
 (segment (start 154.94 93.472) (end 154.649001 93.181001) (width 0.25) (layer B.Cu) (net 7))
 (segment (start 159.512 100.584) (end 154.94 96.012) (width 0.25) (layer B.Cu) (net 7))
 (segment (start 154.94 96.012) (end 154.94 93.472) (width 0.25) (layer B.Cu) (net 7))
 (segment (start 144.78 78.486) (end 144.78 79.756) (width 0.25) (layer F.Cu) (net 7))
 (segment (start 147.147669 76.219753) (end 147.046247 76.219753) (width 0.25) (layer F.Cu) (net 7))
 (segment (start 147.046247 76.219753) (end 144.78 78.486) (width 0.25) (layer F.Cu) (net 7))
 (segment (start 149.243581 75.292419) (end 150.608528 75.292419) (width 0.25) (layer F.Cu) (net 7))
 (segment (start 147.147669 76.219753) (end 148.075003 75.292419) (width 0.25) (layer F.Cu) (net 7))
 (segment (start 148.075003 75.292419) (end 149.243581 75.292419) (width 0.25) (layer F.Cu) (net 7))
 (segment (start 143.675 87.9385) (end 146.05 87.9385) (width 0.25) (layer F.Cu) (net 4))
 (segment (start 142.875 87.9385) (end 143.675 87.9385) (width 0.25) (layer F.Cu) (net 4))
 (segment (start 146.05 87.9385) (end 149.225 87.9385) (width 0.25) (layer F.Cu) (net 4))
 (segment (start 150.025 87.9385) (end 152.4 87.9385) (width 0.25) (layer F.Cu) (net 4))
 (segment (start 149.225 87.9385) (end 150.025 87.9385) (width 0.25) (layer F.Cu) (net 4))
 (segment (start 153.2 87.9385) (end 155.575 87.9385) (width 0.25) (layer F.Cu) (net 4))
 (segment (start 152.4 87.9385) (end 153.2 87.9385) (width 0.25) (layer F.Cu) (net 4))
 (segment (start 155.575 87.9385) (end 158.75 87.9385) (width 0.25) (layer F.Cu) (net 4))
 (segment (start 158.75 87.9385) (end 161.925 87.9385) (width 0.25) (layer F.Cu) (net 4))
 (via (at 156.972 86.36) (size 0.8) (drill 0.4) (layers F.Cu B.Cu) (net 4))
 (segment (start 156.972 86.36) (end 155.956 86.36) (width 0.25) (layer F.Cu) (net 4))
 (segment (start 155.575 86.741) (end 155.575 87.9385) (width 0.25) (layer F.Cu) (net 4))
 (segment (start 155.956 86.36) (end 155.575 86.741) (width 0.25) (layer F.Cu) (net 4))
 (segment (start 156.972 93.98) (end 156.972 86.925685) (width 0.25) (layer B.Cu) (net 4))
 (segment (start 156.972 86.925685) (end 156.972 86.36) (width 0.25) (layer B.Cu) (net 4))
 (segment (start 156.981 103.124) (end 160.02 103.124) (width 0.25) (layer B.Cu) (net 4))
 (segment (start 160.02 103.124) (end 161.036 102.108) (width 0.25) (layer B.Cu) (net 4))
 (segment (start 161.036 98.044) (end 156.972 93.98) (width 0.25) (layer B.Cu) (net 4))
 (segment (start 161.036 102.108) (end 161.036 98.044) (width 0.25) (layer B.Cu) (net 4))
 (segment (start 160.077246 97.592444) (end 161.6624 96.00729) (width 0.25) (layer F.Cu) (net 5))
 (segment (start 159.50729 98.1624) (end 160.077246 97.592444) (width 0.25) (layer F.Cu) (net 5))
 (segment (start 156.079003 100.475119) (end 156.867829 99.686293) (width 0.25) (layer F.Cu) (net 5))
 (segment (start 153.923894 100.475119) (end 156.079003 100.475119) (width 0.25) (layer F.Cu) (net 5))
 (segment (start 157.983397 99.686293) (end 156.867829 99.686293) (width 0.25) (layer F.Cu) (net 5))
 (segment (start 159.50729 98.1624) (end 157.983397 99.686293) (width 0.25) (layer F.Cu) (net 5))
 (segment (start 145.29271 98.1624) (end 143.1376 96.00729) (width 0.25) (layer F.Cu) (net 5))
 (segment (start 154.775 89.9885) (end 152.4 89.9885) (width 0.25) (layer F.Cu) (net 5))
 (segment (start 155.575 89.9885) (end 154.775 89.9885) (width 0.25) (layer F.Cu) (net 5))
 (via (at 146.304 96.52) (size 0.8) (drill 0.4) (layers F.Cu B.Cu) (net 5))
 (segment (start 139.192 96.529) (end 146.295 96.529) (width 0.25) (layer B.Cu) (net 5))
 (segment (start 146.295 96.529) (end 146.304 96.52) (width 0.25) (layer B.Cu) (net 5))
 (segment (start 146.304 97.15111) (end 145.29271 98.1624) (width 0.25) (layer F.Cu) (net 5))
 (segment (start 146.304 96.52) (end 146.304 97.15111) (width 0.25) (layer F.Cu) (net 5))
 (segment (start 161.130001 91.222999) (end 161.6624 91.755398) (width 0.25) (layer F.Cu) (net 5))
 (segment (start 156.809499 91.222999) (end 161.130001 91.222999) (width 0.25) (layer F.Cu) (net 5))
 (segment (start 161.6624 91.755398) (end 161.6624 95.104031) (width 0.25) (layer F.Cu) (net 5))
 (segment (start 161.6624 95.104031) (end 161.6624 96.00729) (width 0.25) (layer F.Cu) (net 5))
 (segment (start 155.575 89.9885) (end 156.809499 91.222999) (width 0.25) (layer F.Cu) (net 5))
 (segment (start 146.195969 98.1624) (end 145.29271 98.1624) (width 0.25) (layer F.Cu) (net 5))
 (segment (start 153.923894 99.567894) (end 152.908 98.552) (width 0.25) (layer F.Cu) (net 5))
 (segment (start 153.923894 100.475119) (end 153.923894 99.567894) (width 0.25) (layer F.Cu) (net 5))
 (segment (start 149.294996 98.552) (end 149.040996 98.298) (width 0.25) (layer F.Cu) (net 5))
 (segment (start 149.040996 98.298) (end 146.331569 98.298) (width 0.25) (layer F.Cu) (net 5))
 (segment (start 152.908 98.552) (end 149.294996 98.552) (width 0.25) (layer F.Cu) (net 5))
 (segment (start 146.331569 98.298) (end 146.195969 98.1624) (width 0.25) (layer F.Cu) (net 5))
 (segment (start 142.081182 97.825206) (end 144.04475 99.788774) (width 0.25) (layer F.Cu) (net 6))
 (segment (start 141.511226 97.25525) (end 142.081182 97.825206) (width 0.25) (layer F.Cu) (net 6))
 (segment (start 145.836223 101.580247) (end 144.04475 99.788774) (width 0.25) (layer F.Cu) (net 6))
 (segment (start 147.147669 101.580247) (end 145.836223 101.580247) (width 0.25) (layer F.Cu) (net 6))
 (segment (start 148.075003 102.507581) (end 150.608528 102.507581) (width 0.25) (layer F.Cu) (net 6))
 (segment (start 147.147669 101.580247) (end 148.075003 102.507581) (width 0.25) (layer F.Cu) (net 6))
 (segment (start 142.875 89.9885) (end 141.511226 91.352274) (width 0.25) (layer F.Cu) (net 6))
 (segment (start 156.079003 77.324881) (end 153.923894 77.324881) (width 0.25) (layer F.Cu) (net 6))
 (segment (start 156.867829 78.113707) (end 156.079003 77.324881) (width 0.25) (layer F.Cu) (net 6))
 (segment (start 141.511226 91.352274) (end 141.511226 91.727226) (width 0.25) (layer F.Cu) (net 6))
 (segment (start 141.511226 91.727226) (end 141.511226 97.25525) (width 0.25) (layer F.Cu) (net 6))
 (via (at 153.924 78.74) (size 0.8) (drill 0.4) (layers F.Cu B.Cu) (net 6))
 (segment (start 153.924 77.324987) (end 153.923894 77.324881) (width 0.25) (layer F.Cu) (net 6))
 (segment (start 153.924 78.74) (end 153.924 77.324987) (width 0.25) (layer F.Cu) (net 6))
 (segment (start 153.924 78.174315) (end 153.924 78.74) (width 0.25) (layer B.Cu) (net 6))
 (segment (start 153.924 75.683) (end 153.924 78.174315) (width 0.25) (layer B.Cu) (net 6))
 (segment (start 152.917 74.676) (end 153.924 75.683) (width 0.25) (layer B.Cu) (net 6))
 (segment (start 141.511226 85.310774) (end 141.511226 91.727226) (width 0.25) (layer F.Cu) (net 6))
 (segment (start 147.624001 79.197999) (end 141.511226 85.310774) (width 0.25) (layer F.Cu) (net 6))
 (segment (start 153.923894 77.324881) (end 152.050776 79.197999) (width 0.25) (layer F.Cu) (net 6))
 (segment (start 152.050776 79.197999) (end 147.624001 79.197999) (width 0.25) (layer F.Cu) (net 6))
 (segment (start 162.061 90.669) (end 161.181999 91.548001) (width 0.25) (layer B.Cu) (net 8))
 (via (at 160.782 91.948) (size 0.8) (drill 0.4) (layers F.Cu B.Cu) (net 8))
 (segment (start 162.061 77.724) (end 162.061 90.669) (width 0.25) (layer B.Cu) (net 8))
 (segment (start 161.181999 91.548001) (end 160.782 91.948) (width 0.25) (layer B.Cu) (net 8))
 (segment (start 157.48 94.742) (end 157.48 96.504) (width 0.25) (layer F.Cu) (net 8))
 (segment (start 158.242 93.98) (end 157.48 94.742) (width 0.25) (layer F.Cu) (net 8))
 (segment (start 159.569679 93.98) (end 158.242 93.98) (width 0.25) (layer F.Cu) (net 8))
 (segment (start 156.575 97.409) (end 156.05 97.409) (width 0.25) (layer F.Cu) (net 8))
 (segment (start 160.782 92.767679) (end 159.569679 93.98) (width 0.25) (layer F.Cu) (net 8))
 (segment (start 160.782 91.948) (end 160.782 92.767679) (width 0.25) (layer F.Cu) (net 8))
 (segment (start 157.48 96.504) (end 156.575 97.409) (width 0.25) (layer F.Cu) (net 8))
 (segment (start 150.876012 97.085685) (end 150.876012 96.52) (width 0.25) (layer B.Cu) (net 9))
 (segment (start 150.876012 101.591012) (end 150.876012 97.085685) (width 0.25) (layer B.Cu) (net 9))
 (via (at 150.876012 96.52) (size 0.8) (drill 0.4) (layers F.Cu B.Cu) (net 9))
 (segment (start 152.409 103.124) (end 150.876012 101.591012) (width 0.25) (layer B.Cu) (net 9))
 (segment (start 154.382 96.52) (end 151.441697 96.52) (width 0.25) (layer F.Cu) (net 9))
 (segment (start 151.441697 96.52) (end 150.876012 96.52) (width 0.25) (layer F.Cu) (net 9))
 (segment (start 154.569 96.52) (end 151.441697 96.52) (width 0.25) (layer F.Cu) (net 9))
 (segment (start 154.95 96.139) (end 154.569 96.52) (width 0.25) (layer F.Cu) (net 9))
 (segment (start 156.05 96.139) (end 154.95 96.139) (width 0.25) (layer F.Cu) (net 9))
 (segment (start 154.931 103.124) (end 153.923993 102.116993) (width 0.25) (layer B.Cu) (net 10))
 (segment (start 153.923993 102.116993) (end 153.923993 96.069692) (width 0.25) (layer B.Cu) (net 10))
 (segment (start 153.923993 96.069692) (end 153.923993 95.504007) (width 0.25) (layer B.Cu) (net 10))
 (segment (start 154.127993 95.504007) (end 153.923993 95.504007) (width 0.25) (layer F.Cu) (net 10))
 (via (at 153.923993 95.504007) (size 0.8) (drill 0.4) (layers F.Cu B.Cu) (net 10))
 (segment (start 154.559 94.869) (end 153.923993 95.504007) (width 0.25) (layer F.Cu) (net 10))
 (segment (start 156.05 94.869) (end 154.559 94.869) (width 0.25) (layer F.Cu) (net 10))
 (via (at 145.287994 94.488) (size 0.8) (drill 0.4) (layers F.Cu B.Cu) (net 11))
 (segment (start 144.887995 94.887999) (end 145.287994 94.488) (width 0.25) (layer B.Cu) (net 11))
 (segment (start 144.779994 94.996) (end 144.887995 94.887999) (width 0.25) (layer B.Cu) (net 11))
 (segment (start 139.192 94.479) (end 139.709 94.996) (width 0.25) (layer B.Cu) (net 11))
 (segment (start 139.709 94.996) (end 144.779994 94.996) (width 0.25) (layer B.Cu) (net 11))
 (segment (start 145.853679 94.488) (end 145.287994 94.488) (width 0.25) (layer F.Cu) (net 11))
 (segment (start 148.75 94.79999) (end 148.43801 94.488) (width 0.25) (layer F.Cu) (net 11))
 (segment (start 148.43801 94.488) (end 145.853679 94.488) (width 0.25) (layer F.Cu) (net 11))
 (segment (start 143.510005 78.485995) (end 143.510005 93.41431) (width 0.25) (layer B.Cu) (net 12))
 (segment (start 150.867 74.676) (end 147.32 74.676) (width 0.25) (layer B.Cu) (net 12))
 (segment (start 146.761 95.25) (end 144.78001 95.25) (width 0.25) (layer F.Cu) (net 12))
 (segment (start 143.510005 93.41431) (end 143.510005 93.979995) (width 0.25) (layer B.Cu) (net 12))
 (segment (start 148.75 96.139) (end 147.65 96.139) (width 0.25) (layer F.Cu) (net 12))
 (segment (start 147.65 96.139) (end 146.761 95.25) (width 0.25) (layer F.Cu) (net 12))
 (segment (start 144.78001 95.25) (end 143.910004 94.379994) (width 0.25) (layer F.Cu) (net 12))
 (segment (start 147.32 74.676) (end 143.510005 78.485995) (width 0.25) (layer B.Cu) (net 12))
 (via (at 143.510005 93.979995) (size 0.8) (drill 0.4) (layers F.Cu B.Cu) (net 12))
 (segment (start 143.910004 94.379994) (end 143.510005 93.979995) (width 0.25) (layer F.Cu) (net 12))
 (segment (start 156.502 80.173) (end 148.552 80.173) (width 0.25) (layer F.Cu) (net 13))
 (via (at 147.32 86.868) (size 0.8) (drill 0.4) (layers F.Cu B.Cu) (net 13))
 (segment (start 147.32 82.305) (end 147.32 86.868) (width 0.25) (layer F.Cu) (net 13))
 (segment (start 148.552 80.173) (end 148.552 81.073) (width 0.25) (layer F.Cu) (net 13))
 (segment (start 148.552 81.073) (end 147.32 82.305) (width 0.25) (layer F.Cu) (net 13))
 (segment (start 147.32 86.868) (end 147.32 92.456) (width 0.25) (layer B.Cu) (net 13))
 (via (at 147.32 92.456) (size 0.8) (drill 0.4) (layers F.Cu B.Cu) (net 13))
 (segment (start 148.68099 93.52999) (end 148.75 93.52999) (width 0.25) (layer F.Cu) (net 13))
 (segment (start 147.607 92.456) (end 148.75 93.599) (width 0.25) (layer F.Cu) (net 13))
 (segment (start 147.32 92.456) (end 147.607 92.456) (width 0.25) (layer F.Cu) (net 13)))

